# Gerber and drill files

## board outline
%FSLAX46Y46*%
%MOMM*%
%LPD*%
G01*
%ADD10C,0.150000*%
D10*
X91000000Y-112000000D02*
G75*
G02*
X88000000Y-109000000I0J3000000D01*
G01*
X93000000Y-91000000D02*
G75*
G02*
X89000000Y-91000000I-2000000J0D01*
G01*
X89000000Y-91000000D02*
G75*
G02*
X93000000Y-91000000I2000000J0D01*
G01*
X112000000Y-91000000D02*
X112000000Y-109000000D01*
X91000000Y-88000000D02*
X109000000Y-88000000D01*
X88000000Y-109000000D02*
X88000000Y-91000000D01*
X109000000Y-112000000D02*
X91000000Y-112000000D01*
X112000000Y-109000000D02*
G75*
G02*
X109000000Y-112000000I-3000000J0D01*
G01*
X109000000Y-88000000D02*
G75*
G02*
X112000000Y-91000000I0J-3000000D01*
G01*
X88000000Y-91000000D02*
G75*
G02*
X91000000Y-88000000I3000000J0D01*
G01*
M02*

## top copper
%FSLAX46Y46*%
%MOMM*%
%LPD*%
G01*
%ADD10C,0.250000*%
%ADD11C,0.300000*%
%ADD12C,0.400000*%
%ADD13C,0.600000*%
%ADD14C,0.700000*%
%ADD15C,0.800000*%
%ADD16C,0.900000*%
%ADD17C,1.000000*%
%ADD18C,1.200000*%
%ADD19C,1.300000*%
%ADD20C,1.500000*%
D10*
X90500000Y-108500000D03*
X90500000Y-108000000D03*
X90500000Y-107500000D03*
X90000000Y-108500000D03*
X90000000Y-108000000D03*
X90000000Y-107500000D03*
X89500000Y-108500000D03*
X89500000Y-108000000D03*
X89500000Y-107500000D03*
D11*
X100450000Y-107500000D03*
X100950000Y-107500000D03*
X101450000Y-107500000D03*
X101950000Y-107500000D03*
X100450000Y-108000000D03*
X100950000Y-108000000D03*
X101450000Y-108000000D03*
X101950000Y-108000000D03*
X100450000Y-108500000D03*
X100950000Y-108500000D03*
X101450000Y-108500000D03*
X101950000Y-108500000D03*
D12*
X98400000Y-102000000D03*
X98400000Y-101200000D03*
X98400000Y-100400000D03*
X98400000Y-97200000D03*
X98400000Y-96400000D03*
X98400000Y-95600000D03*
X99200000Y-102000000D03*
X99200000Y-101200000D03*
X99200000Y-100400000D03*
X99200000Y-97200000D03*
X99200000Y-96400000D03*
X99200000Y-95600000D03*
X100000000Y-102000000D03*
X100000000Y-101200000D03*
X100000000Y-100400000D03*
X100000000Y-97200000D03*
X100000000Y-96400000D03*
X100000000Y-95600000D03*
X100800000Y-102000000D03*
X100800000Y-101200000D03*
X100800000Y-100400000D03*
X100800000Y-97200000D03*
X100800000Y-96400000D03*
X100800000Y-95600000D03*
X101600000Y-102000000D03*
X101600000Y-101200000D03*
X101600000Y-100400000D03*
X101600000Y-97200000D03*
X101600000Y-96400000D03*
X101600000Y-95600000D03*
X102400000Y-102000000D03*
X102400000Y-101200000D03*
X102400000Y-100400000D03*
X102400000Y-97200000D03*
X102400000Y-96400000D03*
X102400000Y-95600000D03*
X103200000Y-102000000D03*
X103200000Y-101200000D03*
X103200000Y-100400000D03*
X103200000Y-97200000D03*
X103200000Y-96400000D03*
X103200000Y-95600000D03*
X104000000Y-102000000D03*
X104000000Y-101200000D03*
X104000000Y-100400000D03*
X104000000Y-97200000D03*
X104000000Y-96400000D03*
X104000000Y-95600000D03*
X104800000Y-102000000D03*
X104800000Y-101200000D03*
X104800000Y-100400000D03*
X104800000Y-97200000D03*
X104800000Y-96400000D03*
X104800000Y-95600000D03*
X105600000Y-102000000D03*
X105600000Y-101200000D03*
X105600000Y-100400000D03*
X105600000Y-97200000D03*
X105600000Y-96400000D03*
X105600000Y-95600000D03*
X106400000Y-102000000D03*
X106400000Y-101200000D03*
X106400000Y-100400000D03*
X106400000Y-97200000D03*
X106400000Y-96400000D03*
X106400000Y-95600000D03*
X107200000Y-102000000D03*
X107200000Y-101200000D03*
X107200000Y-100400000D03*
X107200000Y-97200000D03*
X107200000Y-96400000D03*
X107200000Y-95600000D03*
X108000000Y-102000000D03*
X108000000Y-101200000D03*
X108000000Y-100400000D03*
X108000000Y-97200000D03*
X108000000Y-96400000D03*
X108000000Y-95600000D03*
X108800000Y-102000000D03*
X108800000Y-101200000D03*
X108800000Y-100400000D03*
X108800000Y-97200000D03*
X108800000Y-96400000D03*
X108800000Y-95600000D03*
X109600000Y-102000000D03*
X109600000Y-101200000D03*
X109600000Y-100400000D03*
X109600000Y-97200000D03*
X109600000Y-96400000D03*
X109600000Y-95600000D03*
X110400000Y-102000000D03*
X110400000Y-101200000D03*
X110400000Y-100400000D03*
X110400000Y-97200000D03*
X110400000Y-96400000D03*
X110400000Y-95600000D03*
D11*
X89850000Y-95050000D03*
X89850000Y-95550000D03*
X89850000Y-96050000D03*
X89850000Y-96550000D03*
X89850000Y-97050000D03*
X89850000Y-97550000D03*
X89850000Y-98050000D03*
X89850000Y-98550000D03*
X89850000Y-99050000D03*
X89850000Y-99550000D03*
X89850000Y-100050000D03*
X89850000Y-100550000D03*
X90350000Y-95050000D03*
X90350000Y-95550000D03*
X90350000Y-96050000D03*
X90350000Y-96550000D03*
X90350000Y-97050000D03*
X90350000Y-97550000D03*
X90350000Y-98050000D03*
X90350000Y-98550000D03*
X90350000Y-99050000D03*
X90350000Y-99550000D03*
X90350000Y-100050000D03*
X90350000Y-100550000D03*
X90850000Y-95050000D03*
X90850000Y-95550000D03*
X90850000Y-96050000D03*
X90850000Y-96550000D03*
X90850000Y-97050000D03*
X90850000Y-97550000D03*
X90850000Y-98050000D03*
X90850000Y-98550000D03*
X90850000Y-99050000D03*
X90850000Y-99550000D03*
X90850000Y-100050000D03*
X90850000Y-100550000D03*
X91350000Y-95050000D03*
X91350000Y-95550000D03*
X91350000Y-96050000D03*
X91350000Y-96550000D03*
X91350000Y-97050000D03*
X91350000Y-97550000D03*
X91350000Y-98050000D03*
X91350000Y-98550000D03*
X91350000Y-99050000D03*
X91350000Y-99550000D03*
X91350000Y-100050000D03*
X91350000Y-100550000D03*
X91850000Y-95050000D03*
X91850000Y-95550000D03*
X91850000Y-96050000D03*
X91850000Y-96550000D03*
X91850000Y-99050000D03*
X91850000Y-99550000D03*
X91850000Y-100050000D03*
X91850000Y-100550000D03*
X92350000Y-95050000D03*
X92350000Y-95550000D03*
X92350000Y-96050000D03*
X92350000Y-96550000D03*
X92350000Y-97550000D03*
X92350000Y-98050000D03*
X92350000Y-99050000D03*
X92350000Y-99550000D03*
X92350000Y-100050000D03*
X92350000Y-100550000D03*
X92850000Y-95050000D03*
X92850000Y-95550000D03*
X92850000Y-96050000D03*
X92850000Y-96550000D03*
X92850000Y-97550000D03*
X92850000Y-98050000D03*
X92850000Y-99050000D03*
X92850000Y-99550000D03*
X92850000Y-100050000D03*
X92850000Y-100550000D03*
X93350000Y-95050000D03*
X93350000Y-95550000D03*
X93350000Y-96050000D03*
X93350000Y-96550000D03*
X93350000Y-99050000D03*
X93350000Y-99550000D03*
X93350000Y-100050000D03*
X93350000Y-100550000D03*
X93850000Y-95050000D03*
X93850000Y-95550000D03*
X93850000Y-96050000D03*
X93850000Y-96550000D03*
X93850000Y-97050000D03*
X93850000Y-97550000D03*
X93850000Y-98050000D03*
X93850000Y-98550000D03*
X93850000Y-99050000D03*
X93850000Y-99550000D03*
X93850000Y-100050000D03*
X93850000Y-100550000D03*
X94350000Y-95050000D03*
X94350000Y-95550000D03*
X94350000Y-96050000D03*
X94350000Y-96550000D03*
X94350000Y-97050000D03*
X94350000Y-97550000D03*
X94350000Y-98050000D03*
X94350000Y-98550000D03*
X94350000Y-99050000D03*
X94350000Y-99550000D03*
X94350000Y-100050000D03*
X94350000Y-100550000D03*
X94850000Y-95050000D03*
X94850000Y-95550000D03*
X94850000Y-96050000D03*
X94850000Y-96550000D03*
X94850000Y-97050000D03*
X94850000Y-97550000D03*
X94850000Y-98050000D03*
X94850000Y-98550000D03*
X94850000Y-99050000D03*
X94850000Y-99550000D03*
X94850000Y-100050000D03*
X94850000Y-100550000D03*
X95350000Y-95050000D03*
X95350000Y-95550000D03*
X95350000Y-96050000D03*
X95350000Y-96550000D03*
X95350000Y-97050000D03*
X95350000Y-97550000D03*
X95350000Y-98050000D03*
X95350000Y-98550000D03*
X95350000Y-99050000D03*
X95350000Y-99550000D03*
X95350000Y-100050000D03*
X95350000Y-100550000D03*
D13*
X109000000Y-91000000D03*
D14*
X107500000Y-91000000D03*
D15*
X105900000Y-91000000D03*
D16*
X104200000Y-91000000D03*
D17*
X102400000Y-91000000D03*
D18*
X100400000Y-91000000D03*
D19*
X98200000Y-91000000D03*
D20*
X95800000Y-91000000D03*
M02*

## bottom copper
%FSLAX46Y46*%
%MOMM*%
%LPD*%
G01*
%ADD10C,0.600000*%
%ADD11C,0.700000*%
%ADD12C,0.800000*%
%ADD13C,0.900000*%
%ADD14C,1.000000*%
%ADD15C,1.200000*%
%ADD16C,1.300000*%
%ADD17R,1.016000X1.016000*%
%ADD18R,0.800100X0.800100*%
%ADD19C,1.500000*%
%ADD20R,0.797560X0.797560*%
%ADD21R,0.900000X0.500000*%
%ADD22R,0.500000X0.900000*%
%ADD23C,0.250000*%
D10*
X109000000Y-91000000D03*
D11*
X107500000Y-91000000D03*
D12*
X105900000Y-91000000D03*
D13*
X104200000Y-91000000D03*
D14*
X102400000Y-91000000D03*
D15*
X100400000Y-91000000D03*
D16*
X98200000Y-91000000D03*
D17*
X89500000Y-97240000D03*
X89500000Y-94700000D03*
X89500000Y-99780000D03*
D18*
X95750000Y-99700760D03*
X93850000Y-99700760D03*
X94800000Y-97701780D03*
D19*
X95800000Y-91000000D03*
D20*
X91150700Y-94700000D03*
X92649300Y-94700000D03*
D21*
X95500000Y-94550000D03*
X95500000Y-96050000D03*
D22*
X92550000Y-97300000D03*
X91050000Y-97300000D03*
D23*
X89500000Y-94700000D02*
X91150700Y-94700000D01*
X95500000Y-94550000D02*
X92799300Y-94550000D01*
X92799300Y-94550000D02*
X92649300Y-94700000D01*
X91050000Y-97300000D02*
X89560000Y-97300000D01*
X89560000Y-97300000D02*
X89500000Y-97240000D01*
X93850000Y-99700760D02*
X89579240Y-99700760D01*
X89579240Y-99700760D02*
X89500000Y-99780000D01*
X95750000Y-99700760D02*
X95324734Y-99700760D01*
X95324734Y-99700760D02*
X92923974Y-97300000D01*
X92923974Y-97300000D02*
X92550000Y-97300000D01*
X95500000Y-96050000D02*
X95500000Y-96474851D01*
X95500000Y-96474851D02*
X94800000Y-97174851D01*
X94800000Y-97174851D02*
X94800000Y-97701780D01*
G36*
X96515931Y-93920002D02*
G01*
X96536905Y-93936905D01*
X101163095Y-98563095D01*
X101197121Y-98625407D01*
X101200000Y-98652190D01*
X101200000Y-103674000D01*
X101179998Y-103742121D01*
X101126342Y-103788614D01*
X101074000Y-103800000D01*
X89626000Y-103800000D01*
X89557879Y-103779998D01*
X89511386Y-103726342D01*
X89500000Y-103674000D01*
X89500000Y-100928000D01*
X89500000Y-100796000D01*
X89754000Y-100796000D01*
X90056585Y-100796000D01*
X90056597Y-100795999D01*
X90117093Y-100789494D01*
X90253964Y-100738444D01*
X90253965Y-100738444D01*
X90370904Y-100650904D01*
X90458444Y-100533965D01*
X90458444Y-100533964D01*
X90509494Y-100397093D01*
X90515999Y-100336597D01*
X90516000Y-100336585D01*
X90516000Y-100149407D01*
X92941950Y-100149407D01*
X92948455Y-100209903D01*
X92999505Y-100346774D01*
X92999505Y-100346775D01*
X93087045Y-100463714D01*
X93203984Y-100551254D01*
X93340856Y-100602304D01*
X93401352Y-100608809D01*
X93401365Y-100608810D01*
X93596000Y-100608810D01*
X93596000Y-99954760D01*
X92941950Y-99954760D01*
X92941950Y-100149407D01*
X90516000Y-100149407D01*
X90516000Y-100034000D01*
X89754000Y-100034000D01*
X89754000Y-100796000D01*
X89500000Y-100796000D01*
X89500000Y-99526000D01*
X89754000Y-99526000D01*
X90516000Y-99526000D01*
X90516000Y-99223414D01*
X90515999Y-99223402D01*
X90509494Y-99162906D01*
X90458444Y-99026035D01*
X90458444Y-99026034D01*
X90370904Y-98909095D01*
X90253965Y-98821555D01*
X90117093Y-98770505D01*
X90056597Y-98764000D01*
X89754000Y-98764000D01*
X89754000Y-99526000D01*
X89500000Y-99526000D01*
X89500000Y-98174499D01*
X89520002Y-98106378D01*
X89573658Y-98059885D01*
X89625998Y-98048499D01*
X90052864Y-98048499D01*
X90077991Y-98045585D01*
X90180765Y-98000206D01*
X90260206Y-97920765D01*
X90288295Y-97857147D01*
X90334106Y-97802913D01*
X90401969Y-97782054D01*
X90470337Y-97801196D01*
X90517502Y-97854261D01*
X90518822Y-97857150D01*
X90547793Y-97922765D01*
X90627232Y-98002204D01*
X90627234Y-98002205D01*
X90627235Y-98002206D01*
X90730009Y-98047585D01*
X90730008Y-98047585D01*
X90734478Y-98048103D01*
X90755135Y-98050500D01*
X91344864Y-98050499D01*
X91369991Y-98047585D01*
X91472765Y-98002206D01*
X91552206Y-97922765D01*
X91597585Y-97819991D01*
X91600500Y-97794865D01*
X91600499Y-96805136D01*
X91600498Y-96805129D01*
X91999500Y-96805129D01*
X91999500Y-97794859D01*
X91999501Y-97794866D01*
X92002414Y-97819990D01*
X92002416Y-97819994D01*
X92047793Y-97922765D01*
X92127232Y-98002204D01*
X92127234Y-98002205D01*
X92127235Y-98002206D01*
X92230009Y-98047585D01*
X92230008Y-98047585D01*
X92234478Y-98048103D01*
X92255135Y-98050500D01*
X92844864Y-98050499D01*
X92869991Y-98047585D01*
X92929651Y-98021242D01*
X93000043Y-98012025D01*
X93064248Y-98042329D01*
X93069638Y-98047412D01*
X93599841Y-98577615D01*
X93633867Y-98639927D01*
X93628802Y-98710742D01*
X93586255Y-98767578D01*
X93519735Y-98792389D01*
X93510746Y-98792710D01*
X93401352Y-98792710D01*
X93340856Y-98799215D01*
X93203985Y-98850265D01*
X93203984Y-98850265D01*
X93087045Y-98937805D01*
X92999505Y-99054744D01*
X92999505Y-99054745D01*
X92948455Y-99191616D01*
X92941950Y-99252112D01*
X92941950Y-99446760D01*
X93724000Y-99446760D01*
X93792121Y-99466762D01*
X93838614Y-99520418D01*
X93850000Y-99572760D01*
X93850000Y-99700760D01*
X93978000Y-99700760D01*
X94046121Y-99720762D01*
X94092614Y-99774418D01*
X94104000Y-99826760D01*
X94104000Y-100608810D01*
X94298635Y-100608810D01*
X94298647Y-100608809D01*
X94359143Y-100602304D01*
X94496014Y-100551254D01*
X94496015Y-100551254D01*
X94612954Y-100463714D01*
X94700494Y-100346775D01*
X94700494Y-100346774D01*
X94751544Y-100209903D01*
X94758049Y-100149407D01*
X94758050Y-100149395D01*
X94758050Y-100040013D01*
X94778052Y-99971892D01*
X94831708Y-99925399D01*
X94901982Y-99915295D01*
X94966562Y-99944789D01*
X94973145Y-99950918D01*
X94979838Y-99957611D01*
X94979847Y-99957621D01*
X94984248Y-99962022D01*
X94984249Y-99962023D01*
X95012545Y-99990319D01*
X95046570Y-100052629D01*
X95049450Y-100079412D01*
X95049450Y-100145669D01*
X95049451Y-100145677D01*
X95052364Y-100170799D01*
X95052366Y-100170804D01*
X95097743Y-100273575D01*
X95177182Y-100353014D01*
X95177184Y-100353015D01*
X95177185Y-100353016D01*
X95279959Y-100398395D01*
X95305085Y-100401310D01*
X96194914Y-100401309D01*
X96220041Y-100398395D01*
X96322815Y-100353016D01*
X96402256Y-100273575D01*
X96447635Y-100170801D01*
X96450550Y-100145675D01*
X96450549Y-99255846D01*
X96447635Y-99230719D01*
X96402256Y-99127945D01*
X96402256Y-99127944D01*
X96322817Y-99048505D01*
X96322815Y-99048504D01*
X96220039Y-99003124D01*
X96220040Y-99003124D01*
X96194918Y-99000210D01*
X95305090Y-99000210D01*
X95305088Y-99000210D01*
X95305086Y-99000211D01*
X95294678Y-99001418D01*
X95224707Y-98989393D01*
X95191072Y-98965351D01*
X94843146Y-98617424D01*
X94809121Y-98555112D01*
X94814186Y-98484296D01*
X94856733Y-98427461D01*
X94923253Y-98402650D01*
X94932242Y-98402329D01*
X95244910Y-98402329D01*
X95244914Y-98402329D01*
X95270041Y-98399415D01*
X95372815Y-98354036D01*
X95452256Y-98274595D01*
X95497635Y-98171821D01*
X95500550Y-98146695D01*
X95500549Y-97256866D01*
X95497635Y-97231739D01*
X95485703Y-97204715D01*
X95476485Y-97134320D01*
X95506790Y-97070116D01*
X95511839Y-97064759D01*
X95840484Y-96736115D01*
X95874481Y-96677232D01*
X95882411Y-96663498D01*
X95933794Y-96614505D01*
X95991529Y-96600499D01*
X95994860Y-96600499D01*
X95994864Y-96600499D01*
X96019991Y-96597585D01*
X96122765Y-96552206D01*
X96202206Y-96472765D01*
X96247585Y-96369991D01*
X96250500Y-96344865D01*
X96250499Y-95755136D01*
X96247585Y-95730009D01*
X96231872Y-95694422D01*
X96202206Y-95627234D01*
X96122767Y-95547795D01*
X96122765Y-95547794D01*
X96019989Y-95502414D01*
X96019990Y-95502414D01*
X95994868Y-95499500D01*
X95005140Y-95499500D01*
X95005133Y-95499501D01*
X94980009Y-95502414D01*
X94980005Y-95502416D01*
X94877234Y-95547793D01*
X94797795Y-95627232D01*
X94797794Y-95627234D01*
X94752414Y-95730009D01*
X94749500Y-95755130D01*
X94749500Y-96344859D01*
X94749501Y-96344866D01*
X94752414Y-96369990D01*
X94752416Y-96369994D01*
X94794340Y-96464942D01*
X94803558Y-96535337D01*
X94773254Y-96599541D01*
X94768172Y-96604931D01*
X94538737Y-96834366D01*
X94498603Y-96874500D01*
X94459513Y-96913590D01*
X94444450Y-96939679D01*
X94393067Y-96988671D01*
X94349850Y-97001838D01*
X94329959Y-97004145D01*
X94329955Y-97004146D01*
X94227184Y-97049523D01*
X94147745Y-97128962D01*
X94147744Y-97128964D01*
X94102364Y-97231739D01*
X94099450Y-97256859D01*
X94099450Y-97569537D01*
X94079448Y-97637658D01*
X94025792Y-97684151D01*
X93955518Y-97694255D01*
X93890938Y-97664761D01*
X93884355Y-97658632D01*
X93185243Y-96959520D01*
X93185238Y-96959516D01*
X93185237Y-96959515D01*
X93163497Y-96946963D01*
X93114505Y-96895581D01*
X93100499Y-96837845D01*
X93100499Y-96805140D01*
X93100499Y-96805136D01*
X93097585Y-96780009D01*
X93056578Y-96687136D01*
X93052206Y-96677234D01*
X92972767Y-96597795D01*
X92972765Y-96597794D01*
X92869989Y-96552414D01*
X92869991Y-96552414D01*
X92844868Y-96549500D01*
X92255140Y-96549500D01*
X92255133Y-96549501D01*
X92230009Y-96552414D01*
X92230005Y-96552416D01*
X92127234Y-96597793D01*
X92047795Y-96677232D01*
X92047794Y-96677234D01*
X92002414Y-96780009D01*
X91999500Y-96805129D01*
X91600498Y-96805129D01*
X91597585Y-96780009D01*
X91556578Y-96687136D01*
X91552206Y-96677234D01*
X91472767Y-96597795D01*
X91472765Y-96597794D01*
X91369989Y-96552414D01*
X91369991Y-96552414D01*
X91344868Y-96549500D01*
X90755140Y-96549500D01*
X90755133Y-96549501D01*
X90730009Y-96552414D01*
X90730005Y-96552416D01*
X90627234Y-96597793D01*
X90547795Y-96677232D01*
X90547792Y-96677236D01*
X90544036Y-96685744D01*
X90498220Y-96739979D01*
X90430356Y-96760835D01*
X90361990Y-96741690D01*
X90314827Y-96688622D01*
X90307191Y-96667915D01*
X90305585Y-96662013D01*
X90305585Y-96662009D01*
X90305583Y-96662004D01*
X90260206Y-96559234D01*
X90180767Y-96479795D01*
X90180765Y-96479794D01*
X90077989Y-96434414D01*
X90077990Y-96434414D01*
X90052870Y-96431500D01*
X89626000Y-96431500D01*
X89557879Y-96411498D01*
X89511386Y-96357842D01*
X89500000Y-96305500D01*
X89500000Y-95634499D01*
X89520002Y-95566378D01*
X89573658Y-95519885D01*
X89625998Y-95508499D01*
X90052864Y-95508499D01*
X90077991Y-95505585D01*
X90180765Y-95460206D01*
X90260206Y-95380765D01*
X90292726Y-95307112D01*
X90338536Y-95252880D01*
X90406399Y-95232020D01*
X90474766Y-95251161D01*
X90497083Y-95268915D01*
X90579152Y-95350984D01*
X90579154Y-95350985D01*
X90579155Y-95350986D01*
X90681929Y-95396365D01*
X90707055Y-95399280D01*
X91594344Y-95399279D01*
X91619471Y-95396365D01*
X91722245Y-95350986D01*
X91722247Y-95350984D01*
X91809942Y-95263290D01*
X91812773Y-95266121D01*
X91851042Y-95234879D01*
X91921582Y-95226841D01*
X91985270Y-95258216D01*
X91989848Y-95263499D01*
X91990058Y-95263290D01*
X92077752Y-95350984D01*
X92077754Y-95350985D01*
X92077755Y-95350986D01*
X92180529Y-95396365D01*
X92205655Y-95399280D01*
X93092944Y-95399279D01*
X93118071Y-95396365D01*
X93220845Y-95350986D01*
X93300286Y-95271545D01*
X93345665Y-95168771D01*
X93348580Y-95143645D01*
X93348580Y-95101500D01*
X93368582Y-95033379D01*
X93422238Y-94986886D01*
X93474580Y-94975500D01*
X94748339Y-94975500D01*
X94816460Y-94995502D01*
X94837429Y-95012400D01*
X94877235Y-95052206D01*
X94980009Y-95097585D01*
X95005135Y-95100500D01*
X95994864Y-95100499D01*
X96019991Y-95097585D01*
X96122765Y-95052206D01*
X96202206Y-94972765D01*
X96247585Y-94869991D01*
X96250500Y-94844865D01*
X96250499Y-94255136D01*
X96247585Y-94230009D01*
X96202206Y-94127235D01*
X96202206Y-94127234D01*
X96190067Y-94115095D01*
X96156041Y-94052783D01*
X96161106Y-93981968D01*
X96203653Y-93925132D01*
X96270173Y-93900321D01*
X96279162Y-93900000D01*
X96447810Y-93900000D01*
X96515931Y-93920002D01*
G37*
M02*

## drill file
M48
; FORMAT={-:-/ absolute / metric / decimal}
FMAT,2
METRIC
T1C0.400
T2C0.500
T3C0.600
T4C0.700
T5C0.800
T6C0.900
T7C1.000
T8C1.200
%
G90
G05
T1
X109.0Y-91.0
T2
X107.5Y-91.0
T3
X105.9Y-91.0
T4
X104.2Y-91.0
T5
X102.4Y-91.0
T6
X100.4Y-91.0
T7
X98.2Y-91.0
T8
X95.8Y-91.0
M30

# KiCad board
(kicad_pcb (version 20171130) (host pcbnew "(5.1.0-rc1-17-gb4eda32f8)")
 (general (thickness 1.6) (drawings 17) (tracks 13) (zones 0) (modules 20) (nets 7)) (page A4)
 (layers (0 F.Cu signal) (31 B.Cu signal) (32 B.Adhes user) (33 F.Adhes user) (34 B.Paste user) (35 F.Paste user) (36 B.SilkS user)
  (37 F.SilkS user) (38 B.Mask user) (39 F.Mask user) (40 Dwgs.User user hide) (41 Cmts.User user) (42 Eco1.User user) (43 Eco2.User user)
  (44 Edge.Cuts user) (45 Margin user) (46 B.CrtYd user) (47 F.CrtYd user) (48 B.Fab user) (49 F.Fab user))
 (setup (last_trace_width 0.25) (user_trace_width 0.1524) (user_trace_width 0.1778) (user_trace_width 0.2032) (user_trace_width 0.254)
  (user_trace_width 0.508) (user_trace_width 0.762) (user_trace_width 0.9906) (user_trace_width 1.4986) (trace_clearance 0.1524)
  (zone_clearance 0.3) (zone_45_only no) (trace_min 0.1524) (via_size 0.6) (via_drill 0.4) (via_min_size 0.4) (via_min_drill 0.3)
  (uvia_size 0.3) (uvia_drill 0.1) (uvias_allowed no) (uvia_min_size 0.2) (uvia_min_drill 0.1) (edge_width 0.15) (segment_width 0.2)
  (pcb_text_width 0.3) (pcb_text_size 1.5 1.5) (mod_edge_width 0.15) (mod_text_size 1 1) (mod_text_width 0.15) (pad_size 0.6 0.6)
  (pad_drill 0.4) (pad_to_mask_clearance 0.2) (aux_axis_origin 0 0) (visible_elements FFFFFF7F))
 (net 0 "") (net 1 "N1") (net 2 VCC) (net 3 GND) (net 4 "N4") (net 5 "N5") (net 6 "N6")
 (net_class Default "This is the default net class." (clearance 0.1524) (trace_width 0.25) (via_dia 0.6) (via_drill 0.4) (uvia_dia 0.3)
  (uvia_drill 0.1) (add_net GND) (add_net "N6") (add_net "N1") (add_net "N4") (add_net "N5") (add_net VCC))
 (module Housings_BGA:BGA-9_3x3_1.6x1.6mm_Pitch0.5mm (layer F.Cu) (at 90 108)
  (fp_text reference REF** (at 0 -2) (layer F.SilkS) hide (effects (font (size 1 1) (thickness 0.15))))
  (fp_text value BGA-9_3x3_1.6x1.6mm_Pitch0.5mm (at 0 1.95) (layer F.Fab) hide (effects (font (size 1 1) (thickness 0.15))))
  (pad C3 smd circle (at 0.5 0.5) (size 0.25 0.25) (layers F.Cu F.Paste F.Mask))
  (pad B3 smd circle (at 0.5 0) (size 0.25 0.25) (layers F.Cu F.Paste F.Mask))
  (pad A3 smd circle (at 0.5 -0.5) (size 0.25 0.25) (layers F.Cu F.Paste F.Mask))
  (pad C2 smd circle (at 0 0.5) (size 0.25 0.25) (layers F.Cu F.Paste F.Mask))
  (pad B2 smd circle (at 0 0) (size 0.25 0.25) (layers F.Cu F.Paste F.Mask))
  (pad A2 smd circle (at 0 -0.5) (size 0.25 0.25) (layers F.Cu F.Paste F.Mask))
  (pad C1 smd circle (at -0.5 0.5) (size 0.25 0.25) (layers F.Cu F.Paste F.Mask))
  (pad B1 smd circle (at -0.5 0) (size 0.25 0.25) (layers F.Cu F.Paste F.Mask))
  (pad A1 smd circle (at -0.5 -0.5) (size 0.25 0.25) (layers F.Cu F.Paste F.Mask)))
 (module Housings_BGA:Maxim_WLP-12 (layer F.Cu) (at 101.2 108)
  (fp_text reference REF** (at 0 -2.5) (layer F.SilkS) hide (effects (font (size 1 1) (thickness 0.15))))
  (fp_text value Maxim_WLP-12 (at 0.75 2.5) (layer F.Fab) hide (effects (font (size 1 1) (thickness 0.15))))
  (pad A1 smd circle (at -0.75 -0.5 90) (size 0.3 0.3) (layers F.Cu F.Paste F.Mask))
  (pad A2 smd circle (at -0.25 -0.5 90) (size 0.3 0.3) (layers F.Cu F.Paste F.Mask))
  (pad A3 smd circle (at 0.25 -0.5 90) (size 0.3 0.3) (layers F.Cu F.Paste F.Mask))
  (pad A4 smd circle (at 0.75 -0.5 90) (size 0.3 0.3) (layers F.Cu F.Paste F.Mask))
  (pad B1 smd circle (at -0.75 0 90) (size 0.3 0.3) (layers F.Cu F.Paste F.Mask))
  (pad B2 smd circle (at -0.25 0 90) (size 0.3 0.3) (layers F.Cu F.Paste F.Mask))
  (pad B3 smd circle (at 0.25 0 90) (size 0.3 0.3) (layers F.Cu F.Paste F.Mask))
  (pad B4 smd circle (at 0.75 0 90) (size 0.3 0.3) (layers F.Cu F.Paste F.Mask))
  (pad C1 smd circle (at -0.75 0.5 90) (size 0.3 0.3) (layers F.Cu F.Paste F.Mask))
  (pad C2 smd circle (at -0.25 0.5 90) (size 0.3 0.3) (layers F.Cu F.Paste F.Mask))
  (pad C3 smd circle (at 0.25 0.5 90) (size 0.3 0.3) (layers F.Cu F.Paste F.Mask))
  (pad C4 smd circle (at 0.75 0.5 90) (size 0.3 0.3) (layers F.Cu F.Paste F.Mask)))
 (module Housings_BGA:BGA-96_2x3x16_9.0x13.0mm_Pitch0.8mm (layer F.Cu) (at 104.4 98.8 90)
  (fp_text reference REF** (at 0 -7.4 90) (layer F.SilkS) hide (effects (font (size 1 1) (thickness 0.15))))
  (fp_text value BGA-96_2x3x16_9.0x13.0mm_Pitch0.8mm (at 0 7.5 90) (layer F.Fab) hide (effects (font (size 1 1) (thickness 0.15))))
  (pad A1 smd circle (at -3.2 -6 90) (size 0.4 0.4) (layers F.Cu F.Paste F.Mask))
  (pad A2 smd circle (at -2.4 -6 90) (size 0.4 0.4) (layers F.Cu F.Paste F.Mask))
  (pad A3 smd circle (at -1.6 -6 90) (size 0.4 0.4) (layers F.Cu F.Paste F.Mask))
  (pad A7 smd circle (at 1.6 -6 90) (size 0.4 0.4) (layers F.Cu F.Paste F.Mask))
  (pad A8 smd circle (at 2.4 -6 90) (size 0.4 0.4) (layers F.Cu F.Paste F.Mask))
  (pad A9 smd circle (at 3.2 -6 90) (size 0.4 0.4) (layers F.Cu F.Paste F.Mask))
  (pad B1 smd circle (at -3.2 -5.2 90) (size 0.4 0.4) (layers F.Cu F.Paste F.Mask))
  (pad B2 smd circle (at -2.4 -5.2 90) (size 0.4 0.4) (layers F.Cu F.Paste F.Mask))
  (pad B3 smd circle (at -1.6 -5.2 90) (size 0.4 0.4) (layers F.Cu F.Paste F.Mask))
  (pad B7 smd circle (at 1.6 -5.2 90) (size 0.4 0.4) (layers F.Cu F.Paste F.Mask))
  (pad B8 smd circle (at 2.4 -5.2 90) (size 0.4 0.4) (layers F.Cu F.Paste F.Mask))
  (pad B9 smd circle (at 3.2 -5.2 90) (size 0.4 0.4) (layers F.Cu F.Paste F.Mask))
  (pad C1 smd circle (at -3.2 -4.4 90) (size 0.4 0.4) (layers F.Cu F.Paste F.Mask))
  (pad C2 smd circle (at -2.4 -4.4 90) (size 0.4 0.4) (layers F.Cu F.Paste F.Mask))
  (pad C3 smd circle (at -1.6 -4.4 90) (size 0.4 0.4) (layers F.Cu F.Paste F.Mask))
  (pad C7 smd circle (at 1.6 -4.4 90) (size 0.4 0.4) (layers F.Cu F.Paste F.Mask))
  (pad C8 smd circle (at 2.4 -4.4 90) (size 0.4 0.4) (layers F.Cu F.Paste F.Mask))
  (pad C9 smd circle (at 3.2 -4.4 90) (size 0.4 0.4) (layers F.Cu F.Paste F.Mask))
  (pad D1 smd circle (at -3.2 -3.6 90) (size 0.4 0.4) (layers F.Cu F.Paste F.Mask))
  (pad D2 smd circle (at -2.4 -3.6 90) (size 0.4 0.4) (layers F.Cu F.Paste F.Mask))
  (pad D3 smd circle (at -1.6 -3.6 90) (size 0.4 0.4) (layers F.Cu F.Paste F.Mask))
  (pad D7 smd circle (at 1.6 -3.6 90) (size 0.4 0.4) (layers F.Cu F.Paste F.Mask))
  (pad D8 smd circle (at 2.4 -3.6 90) (size 0.4 0.4) (layers F.Cu F.Paste F.Mask))
  (pad D9 smd circle (at 3.2 -3.6 90) (size 0.4 0.4) (layers F.Cu F.Paste F.Mask))
  (pad E1 smd circle (at -3.2 -2.8 90) (size 0.4 0.4) (layers F.Cu F.Paste F.Mask))
  (pad E2 smd circle (at -2.4 -2.8 90) (size 0.4 0.4) (layers F.Cu F.Paste F.Mask))
  (pad E3 smd circle (at -1.6 -2.8 90) (size 0.4 0.4) (layers F.Cu F.Paste F.Mask))
  (pad E7 smd circle (at 1.6 -2.8 90) (size 0.4 0.4) (layers F.Cu F.Paste F.Mask))
  (pad E8 smd circle (at 2.4 -2.8 90) (size 0.4 0.4) (layers F.Cu F.Paste F.Mask))
  (pad E9 smd circle (at 3.2 -2.8 90) (size 0.4 0.4) (layers F.Cu F.Paste F.Mask))
  (pad F1 smd circle (at -3.2 -2 90) (size 0.4 0.4) (layers F.Cu F.Paste F.Mask))
  (pad F2 smd circle (at -2.4 -2 90) (size 0.4 0.4) (layers F.Cu F.Paste F.Mask))
  (pad F3 smd circle (at -1.6 -2 90) (size 0.4 0.4) (layers F.Cu F.Paste F.Mask))
  (pad F7 smd circle (at 1.6 -2 90) (size 0.4 0.4) (layers F.Cu F.Paste F.Mask))
  (pad F8 smd circle (at 2.4 -2 90) (size 0.4 0.4) (layers F.Cu F.Paste F.Mask))
  (pad F9 smd circle (at 3.2 -2 90) (size 0.4 0.4) (layers F.Cu F.Paste F.Mask))
  (pad G1 smd circle (at -3.2 -1.2 90) (size 0.4 0.4) (layers F.Cu F.Paste F.Mask))
  (pad G2 smd circle (at -2.4 -1.2 90) (size 0.4 0.4) (layers F.Cu F.Paste F.Mask))
  (pad G3 smd circle (at -1.6 -1.2 90) (size 0.4 0.4) (layers F.Cu F.Paste F.Mask))
  (pad G7 smd circle (at 1.6 -1.2 90) (size 0.4 0.4) (layers F.Cu F.Paste F.Mask))
  (pad G8 smd circle (at 2.4 -1.2 90) (size 0.4 0.4) (layers F.Cu F.Paste F.Mask))
  (pad G9 smd circle (at 3.2 -1.2 90) (size 0.4 0.4) (layers F.Cu F.Paste F.Mask))
  (pad H1 smd circle (at -3.2 -0.4 90) (size 0.4 0.4) (layers F.Cu F.Paste F.Mask))
  (pad H2 smd circle (at -2.4 -0.4 90) (size 0.4 0.4) (layers F.Cu F.Paste F.Mask))
  (pad H3 smd circle (at -1.6 -0.4 90) (size 0.4 0.4) (layers F.Cu F.Paste F.Mask))
  (pad H7 smd circle (at 1.6 -0.4 90) (size 0.4 0.4) (layers F.Cu F.Paste F.Mask))
  (pad H8 smd circle (at 2.4 -0.4 90) (size 0.4 0.4) (layers F.Cu F.Paste F.Mask))
  (pad H9 smd circle (at 3.2 -0.4 90) (size 0.4 0.4) (layers F.Cu F.Paste F.Mask))
  (pad J1 smd circle (at -3.2 0.4 90) (size 0.4 0.4) (layers F.Cu F.Paste F.Mask))
  (pad J2 smd circle (at -2.4 0.4 90) (size 0.4 0.4) (layers F.Cu F.Paste F.Mask))
  (pad J3 smd circle (at -1.6 0.4 90) (size 0.4 0.4) (layers F.Cu F.Paste F.Mask))
  (pad J7 smd circle (at 1.6 0.4 90) (size 0.4 0.4) (layers F.Cu F.Paste F.Mask))
  (pad J8 smd circle (at 2.4 0.4 90) (size 0.4 0.4) (layers F.Cu F.Paste F.Mask))
  (pad J9 smd circle (at 3.2 0.4 90) (size 0.4 0.4) (layers F.Cu F.Paste F.Mask))
  (pad K1 smd circle (at -3.2 1.2 90) (size 0.4 0.4) (layers F.Cu F.Paste F.Mask))
  (pad K2 smd circle (at -2.4 1.2 90) (size 0.4 0.4) (layers F.Cu F.Paste F.Mask))
  (pad K3 smd circle (at -1.6 1.2 90) (size 0.4 0.4) (layers F.Cu F.Paste F.Mask))
  (pad K7 smd circle (at 1.6 1.2 90) (size 0.4 0.4) (layers F.Cu F.Paste F.Mask))
  (pad K8 smd circle (at 2.4 1.2 90) (size 0.4 0.4) (layers F.Cu F.Paste F.Mask))
  (pad K9 smd circle (at 3.2 1.2 90) (size 0.4 0.4) (layers F.Cu F.Paste F.Mask))
  (pad L1 smd circle (at -3.2 2 90) (size 0.4 0.4) (layers F.Cu F.Paste F.Mask))
  (pad L2 smd circle (at -2.4 2 90) (size 0.4 0.4) (layers F.Cu F.Paste F.Mask))
  (pad L3 smd circle (at -1.6 2 90) (size 0.4 0.4) (layers F.Cu F.Paste F.Mask))
  (pad L7 smd circle (at 1.6 2 90) (size 0.4 0.4) (layers F.Cu F.Paste F.Mask))
  (pad L8 smd circle (at 2.4 2 90) (size 0.4 0.4) (layers F.Cu F.Paste F.Mask))
  (pad L9 smd circle (at 3.2 2 90) (size 0.4 0.4) (layers F.Cu F.Paste F.Mask))
  (pad M1 smd circle (at -3.2 2.8 90) (size 0.4 0.4) (layers F.Cu F.Paste F.Mask))
  (pad M2 smd circle (at -2.4 2.8 90) (size 0.4 0.4) (layers F.Cu F.Paste F.Mask))
  (pad M3 smd circle (at -1.6 2.8 90) (size 0.4 0.4) (layers F.Cu F.Paste F.Mask))
  (pad M7 smd circle (at 1.6 2.8 90) (size 0.4 0.4) (layers F.Cu F.Paste F.Mask))
  (pad M8 smd circle (at 2.4 2.8 90) (size 0.4 0.4) (layers F.Cu F.Paste F.Mask))
  (pad M9 smd circle (at 3.2 2.8 90) (size 0.4 0.4) (layers F.Cu F.Paste F.Mask))
  (pad N1 smd circle (at -3.2 3.6 90) (size 0.4 0.4) (layers F.Cu F.Paste F.Mask))
  (pad N2 smd circle (at -2.4 3.6 90) (size 0.4 0.4) (layers F.Cu F.Paste F.Mask))
  (pad N3 smd circle (at -1.6 3.6 90) (size 0.4 0.4) (layers F.Cu F.Paste F.Mask))
  (pad N7 smd circle (at 1.6 3.6 90) (size 0.4 0.4) (layers F.Cu F.Paste F.Mask))
  (pad N8 smd circle (at 2.4 3.6 90) (size 0.4 0.4) (layers F.Cu F.Paste F.Mask))
  (pad N9 smd circle (at 3.2 3.6 90) (size 0.4 0.4) (layers F.Cu F.Paste F.Mask))
  (pad P1 smd circle (at -3.2 4.4 90) (size 0.4 0.4) (layers F.Cu F.Paste F.Mask))
  (pad P2 smd circle (at -2.4 4.4 90) (size 0.4 0.4) (layers F.Cu F.Paste F.Mask))
  (pad P3 smd circle (at -1.6 4.4 90) (size 0.4 0.4) (layers F.Cu F.Paste F.Mask))
  (pad P7 smd circle (at 1.6 4.4 90) (size 0.4 0.4) (layers F.Cu F.Paste F.Mask))
  (pad P8 smd circle (at 2.4 4.4 90) (size 0.4 0.4) (layers F.Cu F.Paste F.Mask))
  (pad P9 smd circle (at 3.2 4.4 90) (size 0.4 0.4) (layers F.Cu F.Paste F.Mask))
  (pad R1 smd circle (at -3.2 5.2 90) (size 0.4 0.4) (layers F.Cu F.Paste F.Mask))
  (pad R2 smd circle (at -2.4 5.2 90) (size 0.4 0.4) (layers F.Cu F.Paste F.Mask))
  (pad R3 smd circle (at -1.6 5.2 90) (size 0.4 0.4) (layers F.Cu F.Paste F.Mask))
  (pad R7 smd circle (at 1.6 5.2 90) (size 0.4 0.4) (layers F.Cu F.Paste F.Mask))
  (pad R8 smd circle (at 2.4 5.2 90) (size 0.4 0.4) (layers F.Cu F.Paste F.Mask))
  (pad R9 smd circle (at 3.2 5.2 90) (size 0.4 0.4) (layers F.Cu F.Paste F.Mask))
  (pad T1 smd circle (at -3.2 6 90) (size 0.4 0.4) (layers F.Cu F.Paste F.Mask))
  (pad T2 smd circle (at -2.4 6 90) (size 0.4 0.4) (layers F.Cu F.Paste F.Mask))
  (pad T3 smd circle (at -1.6 6 90) (size 0.4 0.4) (layers F.Cu F.Paste F.Mask))
  (pad T7 smd circle (at 1.6 6 90) (size 0.4 0.4) (layers F.Cu F.Paste F.Mask))
  (pad T8 smd circle (at 2.4 6 90) (size 0.4 0.4) (layers F.Cu F.Paste F.Mask))
  (pad T9 smd circle (at 3.2 6 90) (size 0.4 0.4) (layers F.Cu F.Paste F.Mask)))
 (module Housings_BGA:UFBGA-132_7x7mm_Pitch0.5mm (layer F.Cu) (at 92.6 97.8) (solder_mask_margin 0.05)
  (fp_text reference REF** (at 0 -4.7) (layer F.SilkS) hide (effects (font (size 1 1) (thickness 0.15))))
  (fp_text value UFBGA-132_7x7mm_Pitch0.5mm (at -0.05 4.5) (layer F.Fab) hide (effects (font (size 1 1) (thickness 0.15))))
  (pad A1 smd circle (at -2.75 -2.75) (size 0.3 0.3) (layers F.Cu F.Paste F.Mask))
  (pad B1 smd circle (at -2.75 -2.25) (size 0.3 0.3) (layers F.Cu F.Paste F.Mask))
  (pad C1 smd circle (at -2.75 -1.75) (size 0.3 0.3) (layers F.Cu F.Paste F.Mask))
  (pad D1 smd circle (at -2.75 -1.25) (size 0.3 0.3) (layers F.Cu F.Paste F.Mask))
  (pad E1 smd circle (at -2.75 -0.75) (size 0.3 0.3) (layers F.Cu F.Paste F.Mask))
  (pad F1 smd circle (at -2.75 -0.25) (size 0.3 0.3) (layers F.Cu F.Paste F.Mask))
  (pad G1 smd circle (at -2.75 0.25) (size 0.3 0.3) (layers F.Cu F.Paste F.Mask))
  (pad H1 smd circle (at -2.75 0.75) (size 0.3 0.3) (layers F.Cu F.Paste F.Mask))
  (pad J1 smd circle (at -2.75 1.25) (size 0.3 0.3) (layers F.Cu F.Paste F.Mask))
  (pad K1 smd circle (at -2.75 1.75) (size 0.3 0.3) (layers F.Cu F.Paste F.Mask))
  (pad L1 smd circle (at -2.75 2.25) (size 0.3 0.3) (layers F.Cu F.Paste F.Mask))
  (pad M1 smd circle (at -2.75 2.75) (size 0.3 0.3) (layers F.Cu F.Paste F.Mask))
  (pad A2 smd circle (at -2.25 -2.75) (size 0.3 0.3) (layers F.Cu F.Paste F.Mask))
  (pad B2 smd circle (at -2.25 -2.25) (size 0.3 0.3) (layers F.Cu F.Paste F.Mask))
  (pad C2 smd circle (at -2.25 -1.75) (size 0.3 0.3) (layers F.Cu F.Paste F.Mask))
  (pad D2 smd circle (at -2.25 -1.25) (size 0.3 0.3) (layers F.Cu F.Paste F.Mask))
  (pad E2 smd circle (at -2.25 -0.75) (size 0.3 0.3) (layers F.Cu F.Paste F.Mask))
  (pad F2 smd circle (at -2.25 -0.25) (size 0.3 0.3) (layers F.Cu F.Paste F.Mask))
  (pad G2 smd circle (at -2.25 0.25) (size 0.3 0.3) (layers F.Cu F.Paste F.Mask))
  (pad H2 smd circle (at -2.25 0.75) (size 0.3 0.3) (layers F.Cu F.Paste F.Mask))
  (pad J2 smd circle (at -2.25 1.25) (size 0.3 0.3) (layers F.Cu F.Paste F.Mask))
  (pad K2 smd circle (at -2.25 1.75) (size 0.3 0.3) (layers F.Cu F.Paste F.Mask))
  (pad L2 smd circle (at -2.25 2.25) (size 0.3 0.3) (layers F.Cu F.Paste F.Mask))
  (pad M2 smd circle (at -2.25 2.75) (size 0.3 0.3) (layers F.Cu F.Paste F.Mask))
  (pad A3 smd circle (at -1.75 -2.75) (size 0.3 0.3) (layers F.Cu F.Paste F.Mask))
  (pad B3 smd circle (at -1.75 -2.25) (size 0.3 0.3) (layers F.Cu F.Paste F.Mask))
  (pad C3 smd circle (at -1.75 -1.75) (size 0.3 0.3) (layers F.Cu F.Paste F.Mask))
  (pad D3 smd circle (at -1.75 -1.25) (size 0.3 0.3) (layers F.Cu F.Paste F.Mask))
  (pad E3 smd circle (at -1.75 -0.75) (size 0.3 0.3) (layers F.Cu F.Paste F.Mask))
  (pad F3 smd circle (at -1.75 -0.25) (size 0.3 0.3) (layers F.Cu F.Paste F.Mask))
  (pad G3 smd circle (at -1.75 0.25) (size 0.3 0.3) (layers F.Cu F.Paste F.Mask))
  (pad H3 smd circle (at -1.75 0.75) (size 0.3 0.3) (layers F.Cu F.Paste F.Mask))
  (pad J3 smd circle (at -1.75 1.25) (size 0.3 0.3) (layers F.Cu F.Paste F.Mask))
  (pad K3 smd circle (at -1.75 1.75) (size 0.3 0.3) (layers F.Cu F.Paste F.Mask))
  (pad L3 smd circle (at -1.75 2.25) (size 0.3 0.3) (layers F.Cu F.Paste F.Mask))
  (pad M3 smd circle (at -1.75 2.75) (size 0.3 0.3) (layers F.Cu F.Paste F.Mask))
  (pad A4 smd circle (at -1.25 -2.75) (size 0.3 0.3) (layers F.Cu F.Paste F.Mask))
  (pad B4 smd circle (at -1.25 -2.25) (size 0.3 0.3) (layers F.Cu F.Paste F.Mask))
  (pad C4 smd circle (at -1.25 -1.75) (size 0.3 0.3) (layers F.Cu F.Paste F.Mask))
  (pad D4 smd circle (at -1.25 -1.25) (size 0.3 0.3) (layers F.Cu F.Paste F.Mask))
  (pad E4 smd circle (at -1.25 -0.75) (size 0.3 0.3) (layers F.Cu F.Paste F.Mask))
  (pad F4 smd circle (at -1.25 -0.25) (size 0.3 0.3) (layers F.Cu F.Paste F.Mask))
  (pad G4 smd circle (at -1.25 0.25) (size 0.3 0.3) (layers F.Cu F.Paste F.Mask))
  (pad H4 smd circle (at -1.25 0.75) (size 0.3 0.3) (layers F.Cu F.Paste F.Mask))
  (pad J4 smd circle (at -1.25 1.25) (size 0.3 0.3) (layers F.Cu F.Paste F.Mask))
  (pad K4 smd circle (at -1.25 1.75) (size 0.3 0.3) (layers F.Cu F.Paste F.Mask))
  (pad L4 smd circle (at -1.25 2.25) (size 0.3 0.3) (layers F.Cu F.Paste F.Mask))
  (pad M4 smd circle (at -1.25 2.75) (size 0.3 0.3) (layers F.Cu F.Paste F.Mask))
  (pad A5 smd circle (at -0.75 -2.75) (size 0.3 0.3) (layers F.Cu F.Paste F.Mask))
  (pad B5 smd circle (at -0.75 -2.25) (size 0.3 0.3) (layers F.Cu F.Paste F.Mask))
  (pad C5 smd circle (at -0.75 -1.75) (size 0.3 0.3) (layers F.Cu F.Paste F.Mask))
  (pad D5 smd circle (at -0.75 -1.25) (size 0.3 0.3) (layers F.Cu F.Paste F.Mask))
  (pad J5 smd circle (at -0.75 1.25) (size 0.3 0.3) (layers F.Cu F.Paste F.Mask))
  (pad K5 smd circle (at -0.75 1.75) (size 0.3 0.3) (layers F.Cu F.Paste F.Mask))
  (pad L5 smd circle (at -0.75 2.25) (size 0.3 0.3) (layers F.Cu F.Paste F.Mask))
  (pad M5 smd circle (at -0.75 2.75) (size 0.3 0.3) (layers F.Cu F.Paste F.Mask))
  (pad A6 smd circle (at -0.25 -2.75) (size 0.3 0.3) (layers F.Cu F.Paste F.Mask))
  (pad B6 smd circle (at -0.25 -2.25) (size 0.3 0.3) (layers F.Cu F.Paste F.Mask))
  (pad C6 smd circle (at -0.25 -1.75) (size 0.3 0.3) (layers F.Cu F.Paste F.Mask))
  (pad D6 smd circle (at -0.25 -1.25) (size 0.3 0.3) (layers F.Cu F.Paste F.Mask))
  (pad F6 smd circle (at -0.25 -0.25) (size 0.3 0.3) (layers F.Cu F.Paste F.Mask))
  (pad G6 smd circle (at -0.25 0.25) (size 0.3 0.3) (layers F.Cu F.Paste F.Mask))
  (pad J6 smd circle (at -0.25 1.25) (size 0.3 0.3) (layers F.Cu F.Paste F.Mask))
  (pad K6 smd circle (at -0.25 1.75) (size 0.3 0.3) (layers F.Cu F.Paste F.Mask))
  (pad L6 smd circle (at -0.25 2.25) (size 0.3 0.3) (layers F.Cu F.Paste F.Mask))
  (pad M6 smd circle (at -0.25 2.75) (size 0.3 0.3) (layers F.Cu F.Paste F.Mask))
  (pad A7 smd circle (at 0.25 -2.75) (size 0.3 0.3) (layers F.Cu F.Paste F.Mask))
  (pad B7 smd circle (at 0.25 -2.25) (size 0.3 0.3) (layers F.Cu F.Paste F.Mask))
  (pad C7 smd circle (at 0.25 -1.75) (size 0.3 0.3) (layers F.Cu F.Paste F.Mask))
  (pad D7 smd circle (at 0.25 -1.25) (size 0.3 0.3) (layers F.Cu F.Paste F.Mask))
  (pad F7 smd circle (at 0.25 -0.25) (size 0.3 0.3) (layers F.Cu F.Paste F.Mask))
  (pad G7 smd circle (at 0.25 0.25) (size 0.3 0.3) (layers F.Cu F.Paste F.Mask))
  (pad J7 smd circle (at 0.25 1.25) (size 0.3 0.3) (layers F.Cu F.Paste F.Mask))
  (pad K7 smd circle (at 0.25 1.75) (size 0.3 0.3) (layers F.Cu F.Paste F.Mask))
  (pad L7 smd circle (at 0.25 2.25) (size 0.3 0.3) (layers F.Cu F.Paste F.Mask))
  (pad M7 smd circle (at 0.25 2.75) (size 0.3 0.3) (layers F.Cu F.Paste F.Mask))
  (pad A8 smd circle (at 0.75 -2.75) (size 0.3 0.3) (layers F.Cu F.Paste F.Mask))
  (pad B8 smd circle (at 0.75 -2.25) (size 0.3 0.3) (layers F.Cu F.Paste F.Mask))
  (pad C8 smd circle (at 0.75 -1.75) (size 0.3 0.3) (layers F.Cu F.Paste F.Mask))
  (pad D8 smd circle (at 0.75 -1.25) (size 0.3 0.3) (layers F.Cu F.Paste F.Mask))
  (pad J8 smd circle (at 0.75 1.25) (size 0.3 0.3) (layers F.Cu F.Paste F.Mask))
  (pad K8 smd circle (at 0.75 1.75) (size 0.3 0.3) (layers F.Cu F.Paste F.Mask))
  (pad L8 smd circle (at 0.75 2.25) (size 0.3 0.3) (layers F.Cu F.Paste F.Mask))
  (pad M8 smd circle (at 0.75 2.75) (size 0.3 0.3) (layers F.Cu F.Paste F.Mask))
  (pad A9 smd circle (at 1.25 -2.75) (size 0.3 0.3) (layers F.Cu F.Paste F.Mask))
  (pad B9 smd circle (at 1.25 -2.25) (size 0.3 0.3) (layers F.Cu F.Paste F.Mask))
  (pad C9 smd circle (at 1.25 -1.75) (size 0.3 0.3) (layers F.Cu F.Paste F.Mask))
  (pad D9 smd circle (at 1.25 -1.25) (size 0.3 0.3) (layers F.Cu F.Paste F.Mask))
  (pad E9 smd circle (at 1.25 -0.75) (size 0.3 0.3) (layers F.Cu F.Paste F.Mask))
  (pad F9 smd circle (at 1.25 -0.25) (size 0.3 0.3) (layers F.Cu F.Paste F.Mask))
  (pad G9 smd circle (at 1.25 0.25) (size 0.3 0.3) (layers F.Cu F.Paste F.Mask))
  (pad H9 smd circle (at 1.25 0.75) (size 0.3 0.3) (layers F.Cu F.Paste F.Mask))
  (pad J9 smd circle (at 1.25 1.25) (size 0.3 0.3) (layers F.Cu F.Paste F.Mask))
  (pad K9 smd circle (at 1.25 1.75) (size 0.3 0.3) (layers F.Cu F.Paste F.Mask))
  (pad L9 smd circle (at 1.25 2.25) (size 0.3 0.3) (layers F.Cu F.Paste F.Mask))
  (pad M9 smd circle (at 1.25 2.75) (size 0.3 0.3) (layers F.Cu F.Paste F.Mask))
  (pad A10 smd circle (at 1.75 -2.75) (size 0.3 0.3) (layers F.Cu F.Paste F.Mask))
  (pad B10 smd circle (at 1.75 -2.25) (size 0.3 0.3) (layers F.Cu F.Paste F.Mask))
  (pad C10 smd circle (at 1.75 -1.75) (size 0.3 0.3) (layers F.Cu F.Paste F.Mask))
  (pad D10 smd circle (at 1.75 -1.25) (size 0.3 0.3) (layers F.Cu F.Paste F.Mask))
  (pad E10 smd circle (at 1.75 -0.75) (size 0.3 0.3) (layers F.Cu F.Paste F.Mask))
  (pad F10 smd circle (at 1.75 -0.25) (size 0.3 0.3) (layers F.Cu F.Paste F.Mask))
  (pad G10 smd circle (at 1.75 0.25) (size 0.3 0.3) (layers F.Cu F.Paste F.Mask))
  (pad H10 smd circle (at 1.75 0.75) (size 0.3 0.3) (layers F.Cu F.Paste F.Mask))
  (pad J10 smd circle (at 1.75 1.25) (size 0.3 0.3) (layers F.Cu F.Paste F.Mask))
  (pad K10 smd circle (at 1.75 1.75) (size 0.3 0.3) (layers F.Cu F.Paste F.Mask))
  (pad L10 smd circle (at 1.75 2.25) (size 0.3 0.3) (layers F.Cu F.Paste F.Mask))
  (pad M10 smd circle (at 1.75 2.75) (size 0.3 0.3) (layers F.Cu F.Paste F.Mask))
  (pad A11 smd circle (at 2.25 -2.75) (size 0.3 0.3) (layers F.Cu F.Paste F.Mask))
  (pad B11 smd circle (at 2.25 -2.25) (size 0.3 0.3) (layers F.Cu F.Paste F.Mask))
  (pad C11 smd circle (at 2.25 -1.75) (size 0.3 0.3) (layers F.Cu F.Paste F.Mask))
  (pad D11 smd circle (at 2.25 -1.25) (size 0.3 0.3) (layers F.Cu F.Paste F.Mask))
  (pad E11 smd circle (at 2.25 -0.75) (size 0.3 0.3) (layers F.Cu F.Paste F.Mask))
  (pad F11 smd circle (at 2.25 -0.25) (size 0.3 0.3) (layers F.Cu F.Paste F.Mask))
  (pad G11 smd circle (at 2.25 0.25) (size 0.3 0.3) (layers F.Cu F.Paste F.Mask))
  (pad H11 smd circle (at 2.25 0.75) (size 0.3 0.3) (layers F.Cu F.Paste F.Mask))
  (pad J11 smd circle (at 2.25 1.25) (size 0.3 0.3) (layers F.Cu F.Paste F.Mask))
  (pad K11 smd circle (at 2.25 1.75) (size 0.3 0.3) (layers F.Cu F.Paste F.Mask))
  (pad L11 smd circle (at 2.25 2.25) (size 0.3 0.3) (layers F.Cu F.Paste F.Mask))
  (pad M11 smd circle (at 2.25 2.75) (size 0.3 0.3) (layers F.Cu F.Paste F.Mask))
  (pad A12 smd circle (at 2.75 -2.75) (size 0.3 0.3) (layers F.Cu F.Paste F.Mask))
  (pad B12 smd circle (at 2.75 -2.25) (size 0.3 0.3) (layers F.Cu F.Paste F.Mask))
  (pad C12 smd circle (at 2.75 -1.75) (size 0.3 0.3) (layers F.Cu F.Paste F.Mask))
  (pad D12 smd circle (at 2.75 -1.25) (size 0.3 0.3) (layers F.Cu F.Paste F.Mask))
  (pad E12 smd circle (at 2.75 -0.75) (size 0.3 0.3) (layers F.Cu F.Paste F.Mask))
  (pad F12 smd circle (at 2.75 -0.25) (size 0.3 0.3) (layers F.Cu F.Paste F.Mask))
  (pad G12 smd circle (at 2.75 0.25) (size 0.3 0.3) (layers F.Cu F.Paste F.Mask))
  (pad H12 smd circle (at 2.75 0.75) (size 0.3 0.3) (layers F.Cu F.Paste F.Mask))
  (pad J12 smd circle (at 2.75 1.25) (size 0.3 0.3) (layers F.Cu F.Paste F.Mask))
  (pad K12 smd circle (at 2.75 1.75) (size 0.3 0.3) (layers F.Cu F.Paste F.Mask))
  (pad L12 smd circle (at 2.75 2.25) (size 0.3 0.3) (layers F.Cu F.Paste F.Mask))
  (pad M12 smd circle (at 2.75 2.75) (size 0.3 0.3) (layers F.Cu F.Paste F.Mask)))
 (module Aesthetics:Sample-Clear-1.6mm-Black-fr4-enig (layer B.Cu) (at 100 102.6 180)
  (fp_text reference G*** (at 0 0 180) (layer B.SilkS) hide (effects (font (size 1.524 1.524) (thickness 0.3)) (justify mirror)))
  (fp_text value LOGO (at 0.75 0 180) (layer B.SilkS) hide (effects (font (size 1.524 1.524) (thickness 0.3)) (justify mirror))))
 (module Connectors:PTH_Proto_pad (layer F.Cu) (at 109 91)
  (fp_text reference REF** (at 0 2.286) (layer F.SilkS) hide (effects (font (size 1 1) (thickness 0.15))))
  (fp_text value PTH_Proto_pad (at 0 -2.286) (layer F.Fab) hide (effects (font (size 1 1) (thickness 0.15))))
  (pad 1 thru_hole circle (at 0 0) (size 0.6 0.6) (drill 0.4) (layers *.Cu *.Mask F.SilkS)))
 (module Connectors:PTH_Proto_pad (layer F.Cu) (at 107.5 91)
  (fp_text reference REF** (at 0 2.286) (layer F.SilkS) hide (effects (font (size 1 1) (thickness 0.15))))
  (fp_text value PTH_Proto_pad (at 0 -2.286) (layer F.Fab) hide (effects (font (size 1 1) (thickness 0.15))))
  (pad 1 thru_hole circle (at 0 0) (size 0.7 0.7) (drill 0.5) (layers *.Cu *.Mask F.SilkS)))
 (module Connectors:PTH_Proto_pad (layer F.Cu) (at 105.9 91)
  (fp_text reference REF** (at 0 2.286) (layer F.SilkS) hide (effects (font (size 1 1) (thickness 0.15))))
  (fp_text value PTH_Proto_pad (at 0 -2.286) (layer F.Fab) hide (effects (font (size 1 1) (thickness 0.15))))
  (pad 1 thru_hole circle (at 0 0) (size 0.8 0.8) (drill 0.6) (layers *.Cu *.Mask F.SilkS)))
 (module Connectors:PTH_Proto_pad (layer F.Cu) (at 104.2 91)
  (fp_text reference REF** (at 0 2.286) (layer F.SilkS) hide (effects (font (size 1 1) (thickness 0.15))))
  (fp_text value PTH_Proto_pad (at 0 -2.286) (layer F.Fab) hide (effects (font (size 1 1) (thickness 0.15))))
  (pad 1 thru_hole circle (at 0 0) (size 0.9 0.9) (drill 0.7) (layers *.Cu *.Mask F.SilkS)))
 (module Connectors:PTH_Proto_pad (layer F.Cu) (at 102.4 91)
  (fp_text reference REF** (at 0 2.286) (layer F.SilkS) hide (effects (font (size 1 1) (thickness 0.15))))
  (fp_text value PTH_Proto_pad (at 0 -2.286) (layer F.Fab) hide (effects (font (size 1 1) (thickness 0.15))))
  (pad 1 thru_hole circle (at 0 0) (size 1 1) (drill 0.8) (layers *.Cu *.Mask F.SilkS)))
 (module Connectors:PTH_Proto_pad (layer F.Cu) (at 100.4 91)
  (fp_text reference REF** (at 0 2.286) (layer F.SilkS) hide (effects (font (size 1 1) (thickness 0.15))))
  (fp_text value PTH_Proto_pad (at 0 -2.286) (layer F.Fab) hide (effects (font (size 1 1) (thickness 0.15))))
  (pad 1 thru_hole circle (at 0 0) (size 1.2 1.2) (drill 0.9) (layers *.Cu *.Mask F.SilkS)))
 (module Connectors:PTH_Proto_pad (layer F.Cu) (at 98.2 91)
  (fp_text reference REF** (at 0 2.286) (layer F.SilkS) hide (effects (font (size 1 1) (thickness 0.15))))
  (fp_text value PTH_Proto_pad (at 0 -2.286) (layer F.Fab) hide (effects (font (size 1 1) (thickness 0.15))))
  (pad 1 thru_hole circle (at 0 0) (size 1.3 1.3) (drill 1) (layers *.Cu *.Mask F.SilkS)))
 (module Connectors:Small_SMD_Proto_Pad (layer B.Cu) (at 89.5 97.24)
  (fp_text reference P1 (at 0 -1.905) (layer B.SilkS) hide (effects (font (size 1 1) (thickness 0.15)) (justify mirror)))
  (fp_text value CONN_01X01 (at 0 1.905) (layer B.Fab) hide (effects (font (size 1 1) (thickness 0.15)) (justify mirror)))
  (pad 1 smd rect (at 0 0) (size 1.016 1.016) (layers B.Cu B.Paste B.Mask) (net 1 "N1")))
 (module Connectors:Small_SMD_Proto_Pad (layer B.Cu) (at 89.5 94.7)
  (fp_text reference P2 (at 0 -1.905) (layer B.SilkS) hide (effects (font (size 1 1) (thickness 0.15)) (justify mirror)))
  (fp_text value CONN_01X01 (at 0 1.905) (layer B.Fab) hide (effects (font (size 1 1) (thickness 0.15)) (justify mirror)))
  (pad 1 smd rect (at 0 0) (size 1.016 1.016) (layers B.Cu B.Paste B.Mask) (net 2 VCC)))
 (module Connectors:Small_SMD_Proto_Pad (layer B.Cu) (at 89.5 99.78)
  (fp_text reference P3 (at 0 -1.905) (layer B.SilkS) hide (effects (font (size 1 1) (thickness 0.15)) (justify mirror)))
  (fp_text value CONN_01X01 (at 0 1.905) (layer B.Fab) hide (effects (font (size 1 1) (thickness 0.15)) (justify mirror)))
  (pad 1 smd rect (at 0 0) (size 1.016 1.016) (layers B.Cu B.Paste B.Mask) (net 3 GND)))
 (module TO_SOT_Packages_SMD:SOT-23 (layer B.Cu) (at 94.8 98.7 180)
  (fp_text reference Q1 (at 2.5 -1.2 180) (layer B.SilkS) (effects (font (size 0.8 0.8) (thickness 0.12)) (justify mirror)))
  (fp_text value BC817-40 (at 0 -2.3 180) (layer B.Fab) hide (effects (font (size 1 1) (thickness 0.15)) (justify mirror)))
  (pad 1 smd rect (at -0.95 -1.00076 180) (size 0.8001 0.8001) (layers B.Cu B.Paste B.Mask) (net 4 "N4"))
  (pad 2 smd rect (at 0.95 -1.00076 180) (size 0.8001 0.8001) (layers B.Cu B.Paste B.Mask) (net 3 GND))
  (pad 3 smd rect (at 0 0.99822 180) (size 0.8001 0.8001) (layers B.Cu B.Paste B.Mask) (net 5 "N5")))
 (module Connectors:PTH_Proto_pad (layer F.Cu) (at 95.8 91)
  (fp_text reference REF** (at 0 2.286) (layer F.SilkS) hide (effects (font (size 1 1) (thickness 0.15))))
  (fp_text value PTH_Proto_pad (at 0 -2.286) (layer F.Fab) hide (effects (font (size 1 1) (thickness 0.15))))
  (pad 1 thru_hole circle (at 0 0) (size 1.5 1.5) (drill 1.2) (layers *.Cu *.Mask F.SilkS)))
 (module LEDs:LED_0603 (layer B.Cu) (at 91.9 94.7 180)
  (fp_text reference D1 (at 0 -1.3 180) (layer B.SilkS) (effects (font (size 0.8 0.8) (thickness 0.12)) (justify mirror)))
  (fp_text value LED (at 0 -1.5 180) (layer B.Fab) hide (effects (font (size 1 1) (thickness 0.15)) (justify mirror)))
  (pad 2 smd rect (at 0.7493 0) (size 0.79756 0.79756) (layers B.Cu B.Paste B.Mask) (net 2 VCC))
  (pad 1 smd rect (at -0.7493 0) (size 0.79756 0.79756) (layers B.Cu B.Paste B.Mask) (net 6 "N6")))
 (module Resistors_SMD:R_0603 (layer B.Cu) (at 95.5 95.3 270)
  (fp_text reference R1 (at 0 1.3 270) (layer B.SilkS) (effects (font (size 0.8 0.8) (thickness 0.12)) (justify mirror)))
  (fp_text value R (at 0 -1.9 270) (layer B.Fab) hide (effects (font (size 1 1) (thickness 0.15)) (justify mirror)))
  (pad 1 smd rect (at -0.75 0 270) (size 0.5 0.9) (layers B.Cu B.Paste B.Mask) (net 6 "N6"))
  (pad 2 smd rect (at 0.75 0 270) (size 0.5 0.9) (layers B.Cu B.Paste B.Mask) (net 5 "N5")))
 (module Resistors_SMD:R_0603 (layer B.Cu) (at 91.8 97.3 180)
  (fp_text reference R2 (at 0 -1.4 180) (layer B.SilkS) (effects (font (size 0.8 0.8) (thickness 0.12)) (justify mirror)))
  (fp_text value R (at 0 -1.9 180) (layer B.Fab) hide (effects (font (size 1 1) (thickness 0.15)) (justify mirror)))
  (pad 1 smd rect (at -0.75 0 180) (size 0.5 0.9) (layers B.Cu B.Paste B.Mask) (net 4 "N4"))
  (pad 2 smd rect (at 0.75 0 180) (size 0.5 0.9) (layers B.Cu B.Paste B.Mask) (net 1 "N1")))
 (gr_arc (start 91 109) (end 91 112) (angle 90) (layer Edge.Cuts) (width 0.15))
 (gr_circle (center 91 91) (end 93 91) (layer Edge.Cuts) (width 0.15))
 (gr_line (start 112 91) (end 112 109) (layer Edge.Cuts) (width 0.15))
 (gr_line (start 91 88) (end 109 88) (layer Edge.Cuts) (width 0.15))
 (gr_line (start 88 109) (end 88 91) (layer Edge.Cuts) (width 0.15))
 (gr_line (start 109 112) (end 91 112) (layer Edge.Cuts) (width 0.15))
 (gr_arc (start 109 109) (end 112 109) (angle 90) (layer Edge.Cuts) (width 0.15))
 (gr_arc (start 109 91) (end 109 88) (angle 90) (layer Edge.Cuts) (width 0.15))
 (gr_arc (start 91 91) (end 88 91) (angle 90) (layer Edge.Cuts) (width 0.15))
 (segment (start 89.5 94.7) (end 91.1507 94.7) (width 0.25) (layer B.Cu) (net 2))
 (segment (start 95.5 94.55) (end 92.7993 94.55) (width 0.25) (layer B.Cu) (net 6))
 (segment (start 92.7993 94.55) (end 92.6493 94.7) (width 0.25) (layer B.Cu) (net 6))
 (segment (start 91.05 97.3) (end 89.56 97.3) (width 0.25) (layer B.Cu) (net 1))
 (segment (start 89.56 97.3) (end 89.5 97.24) (width 0.25) (layer B.Cu) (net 1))
 (segment (start 93.85 99.70076) (end 89.57924 99.70076) (width 0.25) (layer B.Cu) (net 3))
 (segment (start 89.57924 99.70076) (end 89.5 99.78) (width 0.25) (layer B.Cu) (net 3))
 (segment (start 95.75 99.70076) (end 95.324734 99.70076) (width 0.25) (layer B.Cu) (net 4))
 (segment (start 95.324734 99.70076) (end 92.923974 97.3) (width 0.25) (layer B.Cu) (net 4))
 (segment (start 92.923974 97.3) (end 92.55 97.3) (width 0.25) (layer B.Cu) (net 4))
 (segment (start 95.5 96.05) (end 95.5 96.474851) (width 0.25) (layer B.Cu) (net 5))
 (segment (start 95.5 96.474851) (end 94.8 97.174851) (width 0.25) (layer B.Cu) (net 5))
 (segment (start 94.8 97.174851) (end 94.8 97.70178) (width 0.25) (layer B.Cu) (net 5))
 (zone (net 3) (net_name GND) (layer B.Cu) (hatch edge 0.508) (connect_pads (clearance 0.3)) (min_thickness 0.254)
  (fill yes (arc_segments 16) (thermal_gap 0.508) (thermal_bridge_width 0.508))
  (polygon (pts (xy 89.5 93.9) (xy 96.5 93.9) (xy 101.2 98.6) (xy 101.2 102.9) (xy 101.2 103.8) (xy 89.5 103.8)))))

